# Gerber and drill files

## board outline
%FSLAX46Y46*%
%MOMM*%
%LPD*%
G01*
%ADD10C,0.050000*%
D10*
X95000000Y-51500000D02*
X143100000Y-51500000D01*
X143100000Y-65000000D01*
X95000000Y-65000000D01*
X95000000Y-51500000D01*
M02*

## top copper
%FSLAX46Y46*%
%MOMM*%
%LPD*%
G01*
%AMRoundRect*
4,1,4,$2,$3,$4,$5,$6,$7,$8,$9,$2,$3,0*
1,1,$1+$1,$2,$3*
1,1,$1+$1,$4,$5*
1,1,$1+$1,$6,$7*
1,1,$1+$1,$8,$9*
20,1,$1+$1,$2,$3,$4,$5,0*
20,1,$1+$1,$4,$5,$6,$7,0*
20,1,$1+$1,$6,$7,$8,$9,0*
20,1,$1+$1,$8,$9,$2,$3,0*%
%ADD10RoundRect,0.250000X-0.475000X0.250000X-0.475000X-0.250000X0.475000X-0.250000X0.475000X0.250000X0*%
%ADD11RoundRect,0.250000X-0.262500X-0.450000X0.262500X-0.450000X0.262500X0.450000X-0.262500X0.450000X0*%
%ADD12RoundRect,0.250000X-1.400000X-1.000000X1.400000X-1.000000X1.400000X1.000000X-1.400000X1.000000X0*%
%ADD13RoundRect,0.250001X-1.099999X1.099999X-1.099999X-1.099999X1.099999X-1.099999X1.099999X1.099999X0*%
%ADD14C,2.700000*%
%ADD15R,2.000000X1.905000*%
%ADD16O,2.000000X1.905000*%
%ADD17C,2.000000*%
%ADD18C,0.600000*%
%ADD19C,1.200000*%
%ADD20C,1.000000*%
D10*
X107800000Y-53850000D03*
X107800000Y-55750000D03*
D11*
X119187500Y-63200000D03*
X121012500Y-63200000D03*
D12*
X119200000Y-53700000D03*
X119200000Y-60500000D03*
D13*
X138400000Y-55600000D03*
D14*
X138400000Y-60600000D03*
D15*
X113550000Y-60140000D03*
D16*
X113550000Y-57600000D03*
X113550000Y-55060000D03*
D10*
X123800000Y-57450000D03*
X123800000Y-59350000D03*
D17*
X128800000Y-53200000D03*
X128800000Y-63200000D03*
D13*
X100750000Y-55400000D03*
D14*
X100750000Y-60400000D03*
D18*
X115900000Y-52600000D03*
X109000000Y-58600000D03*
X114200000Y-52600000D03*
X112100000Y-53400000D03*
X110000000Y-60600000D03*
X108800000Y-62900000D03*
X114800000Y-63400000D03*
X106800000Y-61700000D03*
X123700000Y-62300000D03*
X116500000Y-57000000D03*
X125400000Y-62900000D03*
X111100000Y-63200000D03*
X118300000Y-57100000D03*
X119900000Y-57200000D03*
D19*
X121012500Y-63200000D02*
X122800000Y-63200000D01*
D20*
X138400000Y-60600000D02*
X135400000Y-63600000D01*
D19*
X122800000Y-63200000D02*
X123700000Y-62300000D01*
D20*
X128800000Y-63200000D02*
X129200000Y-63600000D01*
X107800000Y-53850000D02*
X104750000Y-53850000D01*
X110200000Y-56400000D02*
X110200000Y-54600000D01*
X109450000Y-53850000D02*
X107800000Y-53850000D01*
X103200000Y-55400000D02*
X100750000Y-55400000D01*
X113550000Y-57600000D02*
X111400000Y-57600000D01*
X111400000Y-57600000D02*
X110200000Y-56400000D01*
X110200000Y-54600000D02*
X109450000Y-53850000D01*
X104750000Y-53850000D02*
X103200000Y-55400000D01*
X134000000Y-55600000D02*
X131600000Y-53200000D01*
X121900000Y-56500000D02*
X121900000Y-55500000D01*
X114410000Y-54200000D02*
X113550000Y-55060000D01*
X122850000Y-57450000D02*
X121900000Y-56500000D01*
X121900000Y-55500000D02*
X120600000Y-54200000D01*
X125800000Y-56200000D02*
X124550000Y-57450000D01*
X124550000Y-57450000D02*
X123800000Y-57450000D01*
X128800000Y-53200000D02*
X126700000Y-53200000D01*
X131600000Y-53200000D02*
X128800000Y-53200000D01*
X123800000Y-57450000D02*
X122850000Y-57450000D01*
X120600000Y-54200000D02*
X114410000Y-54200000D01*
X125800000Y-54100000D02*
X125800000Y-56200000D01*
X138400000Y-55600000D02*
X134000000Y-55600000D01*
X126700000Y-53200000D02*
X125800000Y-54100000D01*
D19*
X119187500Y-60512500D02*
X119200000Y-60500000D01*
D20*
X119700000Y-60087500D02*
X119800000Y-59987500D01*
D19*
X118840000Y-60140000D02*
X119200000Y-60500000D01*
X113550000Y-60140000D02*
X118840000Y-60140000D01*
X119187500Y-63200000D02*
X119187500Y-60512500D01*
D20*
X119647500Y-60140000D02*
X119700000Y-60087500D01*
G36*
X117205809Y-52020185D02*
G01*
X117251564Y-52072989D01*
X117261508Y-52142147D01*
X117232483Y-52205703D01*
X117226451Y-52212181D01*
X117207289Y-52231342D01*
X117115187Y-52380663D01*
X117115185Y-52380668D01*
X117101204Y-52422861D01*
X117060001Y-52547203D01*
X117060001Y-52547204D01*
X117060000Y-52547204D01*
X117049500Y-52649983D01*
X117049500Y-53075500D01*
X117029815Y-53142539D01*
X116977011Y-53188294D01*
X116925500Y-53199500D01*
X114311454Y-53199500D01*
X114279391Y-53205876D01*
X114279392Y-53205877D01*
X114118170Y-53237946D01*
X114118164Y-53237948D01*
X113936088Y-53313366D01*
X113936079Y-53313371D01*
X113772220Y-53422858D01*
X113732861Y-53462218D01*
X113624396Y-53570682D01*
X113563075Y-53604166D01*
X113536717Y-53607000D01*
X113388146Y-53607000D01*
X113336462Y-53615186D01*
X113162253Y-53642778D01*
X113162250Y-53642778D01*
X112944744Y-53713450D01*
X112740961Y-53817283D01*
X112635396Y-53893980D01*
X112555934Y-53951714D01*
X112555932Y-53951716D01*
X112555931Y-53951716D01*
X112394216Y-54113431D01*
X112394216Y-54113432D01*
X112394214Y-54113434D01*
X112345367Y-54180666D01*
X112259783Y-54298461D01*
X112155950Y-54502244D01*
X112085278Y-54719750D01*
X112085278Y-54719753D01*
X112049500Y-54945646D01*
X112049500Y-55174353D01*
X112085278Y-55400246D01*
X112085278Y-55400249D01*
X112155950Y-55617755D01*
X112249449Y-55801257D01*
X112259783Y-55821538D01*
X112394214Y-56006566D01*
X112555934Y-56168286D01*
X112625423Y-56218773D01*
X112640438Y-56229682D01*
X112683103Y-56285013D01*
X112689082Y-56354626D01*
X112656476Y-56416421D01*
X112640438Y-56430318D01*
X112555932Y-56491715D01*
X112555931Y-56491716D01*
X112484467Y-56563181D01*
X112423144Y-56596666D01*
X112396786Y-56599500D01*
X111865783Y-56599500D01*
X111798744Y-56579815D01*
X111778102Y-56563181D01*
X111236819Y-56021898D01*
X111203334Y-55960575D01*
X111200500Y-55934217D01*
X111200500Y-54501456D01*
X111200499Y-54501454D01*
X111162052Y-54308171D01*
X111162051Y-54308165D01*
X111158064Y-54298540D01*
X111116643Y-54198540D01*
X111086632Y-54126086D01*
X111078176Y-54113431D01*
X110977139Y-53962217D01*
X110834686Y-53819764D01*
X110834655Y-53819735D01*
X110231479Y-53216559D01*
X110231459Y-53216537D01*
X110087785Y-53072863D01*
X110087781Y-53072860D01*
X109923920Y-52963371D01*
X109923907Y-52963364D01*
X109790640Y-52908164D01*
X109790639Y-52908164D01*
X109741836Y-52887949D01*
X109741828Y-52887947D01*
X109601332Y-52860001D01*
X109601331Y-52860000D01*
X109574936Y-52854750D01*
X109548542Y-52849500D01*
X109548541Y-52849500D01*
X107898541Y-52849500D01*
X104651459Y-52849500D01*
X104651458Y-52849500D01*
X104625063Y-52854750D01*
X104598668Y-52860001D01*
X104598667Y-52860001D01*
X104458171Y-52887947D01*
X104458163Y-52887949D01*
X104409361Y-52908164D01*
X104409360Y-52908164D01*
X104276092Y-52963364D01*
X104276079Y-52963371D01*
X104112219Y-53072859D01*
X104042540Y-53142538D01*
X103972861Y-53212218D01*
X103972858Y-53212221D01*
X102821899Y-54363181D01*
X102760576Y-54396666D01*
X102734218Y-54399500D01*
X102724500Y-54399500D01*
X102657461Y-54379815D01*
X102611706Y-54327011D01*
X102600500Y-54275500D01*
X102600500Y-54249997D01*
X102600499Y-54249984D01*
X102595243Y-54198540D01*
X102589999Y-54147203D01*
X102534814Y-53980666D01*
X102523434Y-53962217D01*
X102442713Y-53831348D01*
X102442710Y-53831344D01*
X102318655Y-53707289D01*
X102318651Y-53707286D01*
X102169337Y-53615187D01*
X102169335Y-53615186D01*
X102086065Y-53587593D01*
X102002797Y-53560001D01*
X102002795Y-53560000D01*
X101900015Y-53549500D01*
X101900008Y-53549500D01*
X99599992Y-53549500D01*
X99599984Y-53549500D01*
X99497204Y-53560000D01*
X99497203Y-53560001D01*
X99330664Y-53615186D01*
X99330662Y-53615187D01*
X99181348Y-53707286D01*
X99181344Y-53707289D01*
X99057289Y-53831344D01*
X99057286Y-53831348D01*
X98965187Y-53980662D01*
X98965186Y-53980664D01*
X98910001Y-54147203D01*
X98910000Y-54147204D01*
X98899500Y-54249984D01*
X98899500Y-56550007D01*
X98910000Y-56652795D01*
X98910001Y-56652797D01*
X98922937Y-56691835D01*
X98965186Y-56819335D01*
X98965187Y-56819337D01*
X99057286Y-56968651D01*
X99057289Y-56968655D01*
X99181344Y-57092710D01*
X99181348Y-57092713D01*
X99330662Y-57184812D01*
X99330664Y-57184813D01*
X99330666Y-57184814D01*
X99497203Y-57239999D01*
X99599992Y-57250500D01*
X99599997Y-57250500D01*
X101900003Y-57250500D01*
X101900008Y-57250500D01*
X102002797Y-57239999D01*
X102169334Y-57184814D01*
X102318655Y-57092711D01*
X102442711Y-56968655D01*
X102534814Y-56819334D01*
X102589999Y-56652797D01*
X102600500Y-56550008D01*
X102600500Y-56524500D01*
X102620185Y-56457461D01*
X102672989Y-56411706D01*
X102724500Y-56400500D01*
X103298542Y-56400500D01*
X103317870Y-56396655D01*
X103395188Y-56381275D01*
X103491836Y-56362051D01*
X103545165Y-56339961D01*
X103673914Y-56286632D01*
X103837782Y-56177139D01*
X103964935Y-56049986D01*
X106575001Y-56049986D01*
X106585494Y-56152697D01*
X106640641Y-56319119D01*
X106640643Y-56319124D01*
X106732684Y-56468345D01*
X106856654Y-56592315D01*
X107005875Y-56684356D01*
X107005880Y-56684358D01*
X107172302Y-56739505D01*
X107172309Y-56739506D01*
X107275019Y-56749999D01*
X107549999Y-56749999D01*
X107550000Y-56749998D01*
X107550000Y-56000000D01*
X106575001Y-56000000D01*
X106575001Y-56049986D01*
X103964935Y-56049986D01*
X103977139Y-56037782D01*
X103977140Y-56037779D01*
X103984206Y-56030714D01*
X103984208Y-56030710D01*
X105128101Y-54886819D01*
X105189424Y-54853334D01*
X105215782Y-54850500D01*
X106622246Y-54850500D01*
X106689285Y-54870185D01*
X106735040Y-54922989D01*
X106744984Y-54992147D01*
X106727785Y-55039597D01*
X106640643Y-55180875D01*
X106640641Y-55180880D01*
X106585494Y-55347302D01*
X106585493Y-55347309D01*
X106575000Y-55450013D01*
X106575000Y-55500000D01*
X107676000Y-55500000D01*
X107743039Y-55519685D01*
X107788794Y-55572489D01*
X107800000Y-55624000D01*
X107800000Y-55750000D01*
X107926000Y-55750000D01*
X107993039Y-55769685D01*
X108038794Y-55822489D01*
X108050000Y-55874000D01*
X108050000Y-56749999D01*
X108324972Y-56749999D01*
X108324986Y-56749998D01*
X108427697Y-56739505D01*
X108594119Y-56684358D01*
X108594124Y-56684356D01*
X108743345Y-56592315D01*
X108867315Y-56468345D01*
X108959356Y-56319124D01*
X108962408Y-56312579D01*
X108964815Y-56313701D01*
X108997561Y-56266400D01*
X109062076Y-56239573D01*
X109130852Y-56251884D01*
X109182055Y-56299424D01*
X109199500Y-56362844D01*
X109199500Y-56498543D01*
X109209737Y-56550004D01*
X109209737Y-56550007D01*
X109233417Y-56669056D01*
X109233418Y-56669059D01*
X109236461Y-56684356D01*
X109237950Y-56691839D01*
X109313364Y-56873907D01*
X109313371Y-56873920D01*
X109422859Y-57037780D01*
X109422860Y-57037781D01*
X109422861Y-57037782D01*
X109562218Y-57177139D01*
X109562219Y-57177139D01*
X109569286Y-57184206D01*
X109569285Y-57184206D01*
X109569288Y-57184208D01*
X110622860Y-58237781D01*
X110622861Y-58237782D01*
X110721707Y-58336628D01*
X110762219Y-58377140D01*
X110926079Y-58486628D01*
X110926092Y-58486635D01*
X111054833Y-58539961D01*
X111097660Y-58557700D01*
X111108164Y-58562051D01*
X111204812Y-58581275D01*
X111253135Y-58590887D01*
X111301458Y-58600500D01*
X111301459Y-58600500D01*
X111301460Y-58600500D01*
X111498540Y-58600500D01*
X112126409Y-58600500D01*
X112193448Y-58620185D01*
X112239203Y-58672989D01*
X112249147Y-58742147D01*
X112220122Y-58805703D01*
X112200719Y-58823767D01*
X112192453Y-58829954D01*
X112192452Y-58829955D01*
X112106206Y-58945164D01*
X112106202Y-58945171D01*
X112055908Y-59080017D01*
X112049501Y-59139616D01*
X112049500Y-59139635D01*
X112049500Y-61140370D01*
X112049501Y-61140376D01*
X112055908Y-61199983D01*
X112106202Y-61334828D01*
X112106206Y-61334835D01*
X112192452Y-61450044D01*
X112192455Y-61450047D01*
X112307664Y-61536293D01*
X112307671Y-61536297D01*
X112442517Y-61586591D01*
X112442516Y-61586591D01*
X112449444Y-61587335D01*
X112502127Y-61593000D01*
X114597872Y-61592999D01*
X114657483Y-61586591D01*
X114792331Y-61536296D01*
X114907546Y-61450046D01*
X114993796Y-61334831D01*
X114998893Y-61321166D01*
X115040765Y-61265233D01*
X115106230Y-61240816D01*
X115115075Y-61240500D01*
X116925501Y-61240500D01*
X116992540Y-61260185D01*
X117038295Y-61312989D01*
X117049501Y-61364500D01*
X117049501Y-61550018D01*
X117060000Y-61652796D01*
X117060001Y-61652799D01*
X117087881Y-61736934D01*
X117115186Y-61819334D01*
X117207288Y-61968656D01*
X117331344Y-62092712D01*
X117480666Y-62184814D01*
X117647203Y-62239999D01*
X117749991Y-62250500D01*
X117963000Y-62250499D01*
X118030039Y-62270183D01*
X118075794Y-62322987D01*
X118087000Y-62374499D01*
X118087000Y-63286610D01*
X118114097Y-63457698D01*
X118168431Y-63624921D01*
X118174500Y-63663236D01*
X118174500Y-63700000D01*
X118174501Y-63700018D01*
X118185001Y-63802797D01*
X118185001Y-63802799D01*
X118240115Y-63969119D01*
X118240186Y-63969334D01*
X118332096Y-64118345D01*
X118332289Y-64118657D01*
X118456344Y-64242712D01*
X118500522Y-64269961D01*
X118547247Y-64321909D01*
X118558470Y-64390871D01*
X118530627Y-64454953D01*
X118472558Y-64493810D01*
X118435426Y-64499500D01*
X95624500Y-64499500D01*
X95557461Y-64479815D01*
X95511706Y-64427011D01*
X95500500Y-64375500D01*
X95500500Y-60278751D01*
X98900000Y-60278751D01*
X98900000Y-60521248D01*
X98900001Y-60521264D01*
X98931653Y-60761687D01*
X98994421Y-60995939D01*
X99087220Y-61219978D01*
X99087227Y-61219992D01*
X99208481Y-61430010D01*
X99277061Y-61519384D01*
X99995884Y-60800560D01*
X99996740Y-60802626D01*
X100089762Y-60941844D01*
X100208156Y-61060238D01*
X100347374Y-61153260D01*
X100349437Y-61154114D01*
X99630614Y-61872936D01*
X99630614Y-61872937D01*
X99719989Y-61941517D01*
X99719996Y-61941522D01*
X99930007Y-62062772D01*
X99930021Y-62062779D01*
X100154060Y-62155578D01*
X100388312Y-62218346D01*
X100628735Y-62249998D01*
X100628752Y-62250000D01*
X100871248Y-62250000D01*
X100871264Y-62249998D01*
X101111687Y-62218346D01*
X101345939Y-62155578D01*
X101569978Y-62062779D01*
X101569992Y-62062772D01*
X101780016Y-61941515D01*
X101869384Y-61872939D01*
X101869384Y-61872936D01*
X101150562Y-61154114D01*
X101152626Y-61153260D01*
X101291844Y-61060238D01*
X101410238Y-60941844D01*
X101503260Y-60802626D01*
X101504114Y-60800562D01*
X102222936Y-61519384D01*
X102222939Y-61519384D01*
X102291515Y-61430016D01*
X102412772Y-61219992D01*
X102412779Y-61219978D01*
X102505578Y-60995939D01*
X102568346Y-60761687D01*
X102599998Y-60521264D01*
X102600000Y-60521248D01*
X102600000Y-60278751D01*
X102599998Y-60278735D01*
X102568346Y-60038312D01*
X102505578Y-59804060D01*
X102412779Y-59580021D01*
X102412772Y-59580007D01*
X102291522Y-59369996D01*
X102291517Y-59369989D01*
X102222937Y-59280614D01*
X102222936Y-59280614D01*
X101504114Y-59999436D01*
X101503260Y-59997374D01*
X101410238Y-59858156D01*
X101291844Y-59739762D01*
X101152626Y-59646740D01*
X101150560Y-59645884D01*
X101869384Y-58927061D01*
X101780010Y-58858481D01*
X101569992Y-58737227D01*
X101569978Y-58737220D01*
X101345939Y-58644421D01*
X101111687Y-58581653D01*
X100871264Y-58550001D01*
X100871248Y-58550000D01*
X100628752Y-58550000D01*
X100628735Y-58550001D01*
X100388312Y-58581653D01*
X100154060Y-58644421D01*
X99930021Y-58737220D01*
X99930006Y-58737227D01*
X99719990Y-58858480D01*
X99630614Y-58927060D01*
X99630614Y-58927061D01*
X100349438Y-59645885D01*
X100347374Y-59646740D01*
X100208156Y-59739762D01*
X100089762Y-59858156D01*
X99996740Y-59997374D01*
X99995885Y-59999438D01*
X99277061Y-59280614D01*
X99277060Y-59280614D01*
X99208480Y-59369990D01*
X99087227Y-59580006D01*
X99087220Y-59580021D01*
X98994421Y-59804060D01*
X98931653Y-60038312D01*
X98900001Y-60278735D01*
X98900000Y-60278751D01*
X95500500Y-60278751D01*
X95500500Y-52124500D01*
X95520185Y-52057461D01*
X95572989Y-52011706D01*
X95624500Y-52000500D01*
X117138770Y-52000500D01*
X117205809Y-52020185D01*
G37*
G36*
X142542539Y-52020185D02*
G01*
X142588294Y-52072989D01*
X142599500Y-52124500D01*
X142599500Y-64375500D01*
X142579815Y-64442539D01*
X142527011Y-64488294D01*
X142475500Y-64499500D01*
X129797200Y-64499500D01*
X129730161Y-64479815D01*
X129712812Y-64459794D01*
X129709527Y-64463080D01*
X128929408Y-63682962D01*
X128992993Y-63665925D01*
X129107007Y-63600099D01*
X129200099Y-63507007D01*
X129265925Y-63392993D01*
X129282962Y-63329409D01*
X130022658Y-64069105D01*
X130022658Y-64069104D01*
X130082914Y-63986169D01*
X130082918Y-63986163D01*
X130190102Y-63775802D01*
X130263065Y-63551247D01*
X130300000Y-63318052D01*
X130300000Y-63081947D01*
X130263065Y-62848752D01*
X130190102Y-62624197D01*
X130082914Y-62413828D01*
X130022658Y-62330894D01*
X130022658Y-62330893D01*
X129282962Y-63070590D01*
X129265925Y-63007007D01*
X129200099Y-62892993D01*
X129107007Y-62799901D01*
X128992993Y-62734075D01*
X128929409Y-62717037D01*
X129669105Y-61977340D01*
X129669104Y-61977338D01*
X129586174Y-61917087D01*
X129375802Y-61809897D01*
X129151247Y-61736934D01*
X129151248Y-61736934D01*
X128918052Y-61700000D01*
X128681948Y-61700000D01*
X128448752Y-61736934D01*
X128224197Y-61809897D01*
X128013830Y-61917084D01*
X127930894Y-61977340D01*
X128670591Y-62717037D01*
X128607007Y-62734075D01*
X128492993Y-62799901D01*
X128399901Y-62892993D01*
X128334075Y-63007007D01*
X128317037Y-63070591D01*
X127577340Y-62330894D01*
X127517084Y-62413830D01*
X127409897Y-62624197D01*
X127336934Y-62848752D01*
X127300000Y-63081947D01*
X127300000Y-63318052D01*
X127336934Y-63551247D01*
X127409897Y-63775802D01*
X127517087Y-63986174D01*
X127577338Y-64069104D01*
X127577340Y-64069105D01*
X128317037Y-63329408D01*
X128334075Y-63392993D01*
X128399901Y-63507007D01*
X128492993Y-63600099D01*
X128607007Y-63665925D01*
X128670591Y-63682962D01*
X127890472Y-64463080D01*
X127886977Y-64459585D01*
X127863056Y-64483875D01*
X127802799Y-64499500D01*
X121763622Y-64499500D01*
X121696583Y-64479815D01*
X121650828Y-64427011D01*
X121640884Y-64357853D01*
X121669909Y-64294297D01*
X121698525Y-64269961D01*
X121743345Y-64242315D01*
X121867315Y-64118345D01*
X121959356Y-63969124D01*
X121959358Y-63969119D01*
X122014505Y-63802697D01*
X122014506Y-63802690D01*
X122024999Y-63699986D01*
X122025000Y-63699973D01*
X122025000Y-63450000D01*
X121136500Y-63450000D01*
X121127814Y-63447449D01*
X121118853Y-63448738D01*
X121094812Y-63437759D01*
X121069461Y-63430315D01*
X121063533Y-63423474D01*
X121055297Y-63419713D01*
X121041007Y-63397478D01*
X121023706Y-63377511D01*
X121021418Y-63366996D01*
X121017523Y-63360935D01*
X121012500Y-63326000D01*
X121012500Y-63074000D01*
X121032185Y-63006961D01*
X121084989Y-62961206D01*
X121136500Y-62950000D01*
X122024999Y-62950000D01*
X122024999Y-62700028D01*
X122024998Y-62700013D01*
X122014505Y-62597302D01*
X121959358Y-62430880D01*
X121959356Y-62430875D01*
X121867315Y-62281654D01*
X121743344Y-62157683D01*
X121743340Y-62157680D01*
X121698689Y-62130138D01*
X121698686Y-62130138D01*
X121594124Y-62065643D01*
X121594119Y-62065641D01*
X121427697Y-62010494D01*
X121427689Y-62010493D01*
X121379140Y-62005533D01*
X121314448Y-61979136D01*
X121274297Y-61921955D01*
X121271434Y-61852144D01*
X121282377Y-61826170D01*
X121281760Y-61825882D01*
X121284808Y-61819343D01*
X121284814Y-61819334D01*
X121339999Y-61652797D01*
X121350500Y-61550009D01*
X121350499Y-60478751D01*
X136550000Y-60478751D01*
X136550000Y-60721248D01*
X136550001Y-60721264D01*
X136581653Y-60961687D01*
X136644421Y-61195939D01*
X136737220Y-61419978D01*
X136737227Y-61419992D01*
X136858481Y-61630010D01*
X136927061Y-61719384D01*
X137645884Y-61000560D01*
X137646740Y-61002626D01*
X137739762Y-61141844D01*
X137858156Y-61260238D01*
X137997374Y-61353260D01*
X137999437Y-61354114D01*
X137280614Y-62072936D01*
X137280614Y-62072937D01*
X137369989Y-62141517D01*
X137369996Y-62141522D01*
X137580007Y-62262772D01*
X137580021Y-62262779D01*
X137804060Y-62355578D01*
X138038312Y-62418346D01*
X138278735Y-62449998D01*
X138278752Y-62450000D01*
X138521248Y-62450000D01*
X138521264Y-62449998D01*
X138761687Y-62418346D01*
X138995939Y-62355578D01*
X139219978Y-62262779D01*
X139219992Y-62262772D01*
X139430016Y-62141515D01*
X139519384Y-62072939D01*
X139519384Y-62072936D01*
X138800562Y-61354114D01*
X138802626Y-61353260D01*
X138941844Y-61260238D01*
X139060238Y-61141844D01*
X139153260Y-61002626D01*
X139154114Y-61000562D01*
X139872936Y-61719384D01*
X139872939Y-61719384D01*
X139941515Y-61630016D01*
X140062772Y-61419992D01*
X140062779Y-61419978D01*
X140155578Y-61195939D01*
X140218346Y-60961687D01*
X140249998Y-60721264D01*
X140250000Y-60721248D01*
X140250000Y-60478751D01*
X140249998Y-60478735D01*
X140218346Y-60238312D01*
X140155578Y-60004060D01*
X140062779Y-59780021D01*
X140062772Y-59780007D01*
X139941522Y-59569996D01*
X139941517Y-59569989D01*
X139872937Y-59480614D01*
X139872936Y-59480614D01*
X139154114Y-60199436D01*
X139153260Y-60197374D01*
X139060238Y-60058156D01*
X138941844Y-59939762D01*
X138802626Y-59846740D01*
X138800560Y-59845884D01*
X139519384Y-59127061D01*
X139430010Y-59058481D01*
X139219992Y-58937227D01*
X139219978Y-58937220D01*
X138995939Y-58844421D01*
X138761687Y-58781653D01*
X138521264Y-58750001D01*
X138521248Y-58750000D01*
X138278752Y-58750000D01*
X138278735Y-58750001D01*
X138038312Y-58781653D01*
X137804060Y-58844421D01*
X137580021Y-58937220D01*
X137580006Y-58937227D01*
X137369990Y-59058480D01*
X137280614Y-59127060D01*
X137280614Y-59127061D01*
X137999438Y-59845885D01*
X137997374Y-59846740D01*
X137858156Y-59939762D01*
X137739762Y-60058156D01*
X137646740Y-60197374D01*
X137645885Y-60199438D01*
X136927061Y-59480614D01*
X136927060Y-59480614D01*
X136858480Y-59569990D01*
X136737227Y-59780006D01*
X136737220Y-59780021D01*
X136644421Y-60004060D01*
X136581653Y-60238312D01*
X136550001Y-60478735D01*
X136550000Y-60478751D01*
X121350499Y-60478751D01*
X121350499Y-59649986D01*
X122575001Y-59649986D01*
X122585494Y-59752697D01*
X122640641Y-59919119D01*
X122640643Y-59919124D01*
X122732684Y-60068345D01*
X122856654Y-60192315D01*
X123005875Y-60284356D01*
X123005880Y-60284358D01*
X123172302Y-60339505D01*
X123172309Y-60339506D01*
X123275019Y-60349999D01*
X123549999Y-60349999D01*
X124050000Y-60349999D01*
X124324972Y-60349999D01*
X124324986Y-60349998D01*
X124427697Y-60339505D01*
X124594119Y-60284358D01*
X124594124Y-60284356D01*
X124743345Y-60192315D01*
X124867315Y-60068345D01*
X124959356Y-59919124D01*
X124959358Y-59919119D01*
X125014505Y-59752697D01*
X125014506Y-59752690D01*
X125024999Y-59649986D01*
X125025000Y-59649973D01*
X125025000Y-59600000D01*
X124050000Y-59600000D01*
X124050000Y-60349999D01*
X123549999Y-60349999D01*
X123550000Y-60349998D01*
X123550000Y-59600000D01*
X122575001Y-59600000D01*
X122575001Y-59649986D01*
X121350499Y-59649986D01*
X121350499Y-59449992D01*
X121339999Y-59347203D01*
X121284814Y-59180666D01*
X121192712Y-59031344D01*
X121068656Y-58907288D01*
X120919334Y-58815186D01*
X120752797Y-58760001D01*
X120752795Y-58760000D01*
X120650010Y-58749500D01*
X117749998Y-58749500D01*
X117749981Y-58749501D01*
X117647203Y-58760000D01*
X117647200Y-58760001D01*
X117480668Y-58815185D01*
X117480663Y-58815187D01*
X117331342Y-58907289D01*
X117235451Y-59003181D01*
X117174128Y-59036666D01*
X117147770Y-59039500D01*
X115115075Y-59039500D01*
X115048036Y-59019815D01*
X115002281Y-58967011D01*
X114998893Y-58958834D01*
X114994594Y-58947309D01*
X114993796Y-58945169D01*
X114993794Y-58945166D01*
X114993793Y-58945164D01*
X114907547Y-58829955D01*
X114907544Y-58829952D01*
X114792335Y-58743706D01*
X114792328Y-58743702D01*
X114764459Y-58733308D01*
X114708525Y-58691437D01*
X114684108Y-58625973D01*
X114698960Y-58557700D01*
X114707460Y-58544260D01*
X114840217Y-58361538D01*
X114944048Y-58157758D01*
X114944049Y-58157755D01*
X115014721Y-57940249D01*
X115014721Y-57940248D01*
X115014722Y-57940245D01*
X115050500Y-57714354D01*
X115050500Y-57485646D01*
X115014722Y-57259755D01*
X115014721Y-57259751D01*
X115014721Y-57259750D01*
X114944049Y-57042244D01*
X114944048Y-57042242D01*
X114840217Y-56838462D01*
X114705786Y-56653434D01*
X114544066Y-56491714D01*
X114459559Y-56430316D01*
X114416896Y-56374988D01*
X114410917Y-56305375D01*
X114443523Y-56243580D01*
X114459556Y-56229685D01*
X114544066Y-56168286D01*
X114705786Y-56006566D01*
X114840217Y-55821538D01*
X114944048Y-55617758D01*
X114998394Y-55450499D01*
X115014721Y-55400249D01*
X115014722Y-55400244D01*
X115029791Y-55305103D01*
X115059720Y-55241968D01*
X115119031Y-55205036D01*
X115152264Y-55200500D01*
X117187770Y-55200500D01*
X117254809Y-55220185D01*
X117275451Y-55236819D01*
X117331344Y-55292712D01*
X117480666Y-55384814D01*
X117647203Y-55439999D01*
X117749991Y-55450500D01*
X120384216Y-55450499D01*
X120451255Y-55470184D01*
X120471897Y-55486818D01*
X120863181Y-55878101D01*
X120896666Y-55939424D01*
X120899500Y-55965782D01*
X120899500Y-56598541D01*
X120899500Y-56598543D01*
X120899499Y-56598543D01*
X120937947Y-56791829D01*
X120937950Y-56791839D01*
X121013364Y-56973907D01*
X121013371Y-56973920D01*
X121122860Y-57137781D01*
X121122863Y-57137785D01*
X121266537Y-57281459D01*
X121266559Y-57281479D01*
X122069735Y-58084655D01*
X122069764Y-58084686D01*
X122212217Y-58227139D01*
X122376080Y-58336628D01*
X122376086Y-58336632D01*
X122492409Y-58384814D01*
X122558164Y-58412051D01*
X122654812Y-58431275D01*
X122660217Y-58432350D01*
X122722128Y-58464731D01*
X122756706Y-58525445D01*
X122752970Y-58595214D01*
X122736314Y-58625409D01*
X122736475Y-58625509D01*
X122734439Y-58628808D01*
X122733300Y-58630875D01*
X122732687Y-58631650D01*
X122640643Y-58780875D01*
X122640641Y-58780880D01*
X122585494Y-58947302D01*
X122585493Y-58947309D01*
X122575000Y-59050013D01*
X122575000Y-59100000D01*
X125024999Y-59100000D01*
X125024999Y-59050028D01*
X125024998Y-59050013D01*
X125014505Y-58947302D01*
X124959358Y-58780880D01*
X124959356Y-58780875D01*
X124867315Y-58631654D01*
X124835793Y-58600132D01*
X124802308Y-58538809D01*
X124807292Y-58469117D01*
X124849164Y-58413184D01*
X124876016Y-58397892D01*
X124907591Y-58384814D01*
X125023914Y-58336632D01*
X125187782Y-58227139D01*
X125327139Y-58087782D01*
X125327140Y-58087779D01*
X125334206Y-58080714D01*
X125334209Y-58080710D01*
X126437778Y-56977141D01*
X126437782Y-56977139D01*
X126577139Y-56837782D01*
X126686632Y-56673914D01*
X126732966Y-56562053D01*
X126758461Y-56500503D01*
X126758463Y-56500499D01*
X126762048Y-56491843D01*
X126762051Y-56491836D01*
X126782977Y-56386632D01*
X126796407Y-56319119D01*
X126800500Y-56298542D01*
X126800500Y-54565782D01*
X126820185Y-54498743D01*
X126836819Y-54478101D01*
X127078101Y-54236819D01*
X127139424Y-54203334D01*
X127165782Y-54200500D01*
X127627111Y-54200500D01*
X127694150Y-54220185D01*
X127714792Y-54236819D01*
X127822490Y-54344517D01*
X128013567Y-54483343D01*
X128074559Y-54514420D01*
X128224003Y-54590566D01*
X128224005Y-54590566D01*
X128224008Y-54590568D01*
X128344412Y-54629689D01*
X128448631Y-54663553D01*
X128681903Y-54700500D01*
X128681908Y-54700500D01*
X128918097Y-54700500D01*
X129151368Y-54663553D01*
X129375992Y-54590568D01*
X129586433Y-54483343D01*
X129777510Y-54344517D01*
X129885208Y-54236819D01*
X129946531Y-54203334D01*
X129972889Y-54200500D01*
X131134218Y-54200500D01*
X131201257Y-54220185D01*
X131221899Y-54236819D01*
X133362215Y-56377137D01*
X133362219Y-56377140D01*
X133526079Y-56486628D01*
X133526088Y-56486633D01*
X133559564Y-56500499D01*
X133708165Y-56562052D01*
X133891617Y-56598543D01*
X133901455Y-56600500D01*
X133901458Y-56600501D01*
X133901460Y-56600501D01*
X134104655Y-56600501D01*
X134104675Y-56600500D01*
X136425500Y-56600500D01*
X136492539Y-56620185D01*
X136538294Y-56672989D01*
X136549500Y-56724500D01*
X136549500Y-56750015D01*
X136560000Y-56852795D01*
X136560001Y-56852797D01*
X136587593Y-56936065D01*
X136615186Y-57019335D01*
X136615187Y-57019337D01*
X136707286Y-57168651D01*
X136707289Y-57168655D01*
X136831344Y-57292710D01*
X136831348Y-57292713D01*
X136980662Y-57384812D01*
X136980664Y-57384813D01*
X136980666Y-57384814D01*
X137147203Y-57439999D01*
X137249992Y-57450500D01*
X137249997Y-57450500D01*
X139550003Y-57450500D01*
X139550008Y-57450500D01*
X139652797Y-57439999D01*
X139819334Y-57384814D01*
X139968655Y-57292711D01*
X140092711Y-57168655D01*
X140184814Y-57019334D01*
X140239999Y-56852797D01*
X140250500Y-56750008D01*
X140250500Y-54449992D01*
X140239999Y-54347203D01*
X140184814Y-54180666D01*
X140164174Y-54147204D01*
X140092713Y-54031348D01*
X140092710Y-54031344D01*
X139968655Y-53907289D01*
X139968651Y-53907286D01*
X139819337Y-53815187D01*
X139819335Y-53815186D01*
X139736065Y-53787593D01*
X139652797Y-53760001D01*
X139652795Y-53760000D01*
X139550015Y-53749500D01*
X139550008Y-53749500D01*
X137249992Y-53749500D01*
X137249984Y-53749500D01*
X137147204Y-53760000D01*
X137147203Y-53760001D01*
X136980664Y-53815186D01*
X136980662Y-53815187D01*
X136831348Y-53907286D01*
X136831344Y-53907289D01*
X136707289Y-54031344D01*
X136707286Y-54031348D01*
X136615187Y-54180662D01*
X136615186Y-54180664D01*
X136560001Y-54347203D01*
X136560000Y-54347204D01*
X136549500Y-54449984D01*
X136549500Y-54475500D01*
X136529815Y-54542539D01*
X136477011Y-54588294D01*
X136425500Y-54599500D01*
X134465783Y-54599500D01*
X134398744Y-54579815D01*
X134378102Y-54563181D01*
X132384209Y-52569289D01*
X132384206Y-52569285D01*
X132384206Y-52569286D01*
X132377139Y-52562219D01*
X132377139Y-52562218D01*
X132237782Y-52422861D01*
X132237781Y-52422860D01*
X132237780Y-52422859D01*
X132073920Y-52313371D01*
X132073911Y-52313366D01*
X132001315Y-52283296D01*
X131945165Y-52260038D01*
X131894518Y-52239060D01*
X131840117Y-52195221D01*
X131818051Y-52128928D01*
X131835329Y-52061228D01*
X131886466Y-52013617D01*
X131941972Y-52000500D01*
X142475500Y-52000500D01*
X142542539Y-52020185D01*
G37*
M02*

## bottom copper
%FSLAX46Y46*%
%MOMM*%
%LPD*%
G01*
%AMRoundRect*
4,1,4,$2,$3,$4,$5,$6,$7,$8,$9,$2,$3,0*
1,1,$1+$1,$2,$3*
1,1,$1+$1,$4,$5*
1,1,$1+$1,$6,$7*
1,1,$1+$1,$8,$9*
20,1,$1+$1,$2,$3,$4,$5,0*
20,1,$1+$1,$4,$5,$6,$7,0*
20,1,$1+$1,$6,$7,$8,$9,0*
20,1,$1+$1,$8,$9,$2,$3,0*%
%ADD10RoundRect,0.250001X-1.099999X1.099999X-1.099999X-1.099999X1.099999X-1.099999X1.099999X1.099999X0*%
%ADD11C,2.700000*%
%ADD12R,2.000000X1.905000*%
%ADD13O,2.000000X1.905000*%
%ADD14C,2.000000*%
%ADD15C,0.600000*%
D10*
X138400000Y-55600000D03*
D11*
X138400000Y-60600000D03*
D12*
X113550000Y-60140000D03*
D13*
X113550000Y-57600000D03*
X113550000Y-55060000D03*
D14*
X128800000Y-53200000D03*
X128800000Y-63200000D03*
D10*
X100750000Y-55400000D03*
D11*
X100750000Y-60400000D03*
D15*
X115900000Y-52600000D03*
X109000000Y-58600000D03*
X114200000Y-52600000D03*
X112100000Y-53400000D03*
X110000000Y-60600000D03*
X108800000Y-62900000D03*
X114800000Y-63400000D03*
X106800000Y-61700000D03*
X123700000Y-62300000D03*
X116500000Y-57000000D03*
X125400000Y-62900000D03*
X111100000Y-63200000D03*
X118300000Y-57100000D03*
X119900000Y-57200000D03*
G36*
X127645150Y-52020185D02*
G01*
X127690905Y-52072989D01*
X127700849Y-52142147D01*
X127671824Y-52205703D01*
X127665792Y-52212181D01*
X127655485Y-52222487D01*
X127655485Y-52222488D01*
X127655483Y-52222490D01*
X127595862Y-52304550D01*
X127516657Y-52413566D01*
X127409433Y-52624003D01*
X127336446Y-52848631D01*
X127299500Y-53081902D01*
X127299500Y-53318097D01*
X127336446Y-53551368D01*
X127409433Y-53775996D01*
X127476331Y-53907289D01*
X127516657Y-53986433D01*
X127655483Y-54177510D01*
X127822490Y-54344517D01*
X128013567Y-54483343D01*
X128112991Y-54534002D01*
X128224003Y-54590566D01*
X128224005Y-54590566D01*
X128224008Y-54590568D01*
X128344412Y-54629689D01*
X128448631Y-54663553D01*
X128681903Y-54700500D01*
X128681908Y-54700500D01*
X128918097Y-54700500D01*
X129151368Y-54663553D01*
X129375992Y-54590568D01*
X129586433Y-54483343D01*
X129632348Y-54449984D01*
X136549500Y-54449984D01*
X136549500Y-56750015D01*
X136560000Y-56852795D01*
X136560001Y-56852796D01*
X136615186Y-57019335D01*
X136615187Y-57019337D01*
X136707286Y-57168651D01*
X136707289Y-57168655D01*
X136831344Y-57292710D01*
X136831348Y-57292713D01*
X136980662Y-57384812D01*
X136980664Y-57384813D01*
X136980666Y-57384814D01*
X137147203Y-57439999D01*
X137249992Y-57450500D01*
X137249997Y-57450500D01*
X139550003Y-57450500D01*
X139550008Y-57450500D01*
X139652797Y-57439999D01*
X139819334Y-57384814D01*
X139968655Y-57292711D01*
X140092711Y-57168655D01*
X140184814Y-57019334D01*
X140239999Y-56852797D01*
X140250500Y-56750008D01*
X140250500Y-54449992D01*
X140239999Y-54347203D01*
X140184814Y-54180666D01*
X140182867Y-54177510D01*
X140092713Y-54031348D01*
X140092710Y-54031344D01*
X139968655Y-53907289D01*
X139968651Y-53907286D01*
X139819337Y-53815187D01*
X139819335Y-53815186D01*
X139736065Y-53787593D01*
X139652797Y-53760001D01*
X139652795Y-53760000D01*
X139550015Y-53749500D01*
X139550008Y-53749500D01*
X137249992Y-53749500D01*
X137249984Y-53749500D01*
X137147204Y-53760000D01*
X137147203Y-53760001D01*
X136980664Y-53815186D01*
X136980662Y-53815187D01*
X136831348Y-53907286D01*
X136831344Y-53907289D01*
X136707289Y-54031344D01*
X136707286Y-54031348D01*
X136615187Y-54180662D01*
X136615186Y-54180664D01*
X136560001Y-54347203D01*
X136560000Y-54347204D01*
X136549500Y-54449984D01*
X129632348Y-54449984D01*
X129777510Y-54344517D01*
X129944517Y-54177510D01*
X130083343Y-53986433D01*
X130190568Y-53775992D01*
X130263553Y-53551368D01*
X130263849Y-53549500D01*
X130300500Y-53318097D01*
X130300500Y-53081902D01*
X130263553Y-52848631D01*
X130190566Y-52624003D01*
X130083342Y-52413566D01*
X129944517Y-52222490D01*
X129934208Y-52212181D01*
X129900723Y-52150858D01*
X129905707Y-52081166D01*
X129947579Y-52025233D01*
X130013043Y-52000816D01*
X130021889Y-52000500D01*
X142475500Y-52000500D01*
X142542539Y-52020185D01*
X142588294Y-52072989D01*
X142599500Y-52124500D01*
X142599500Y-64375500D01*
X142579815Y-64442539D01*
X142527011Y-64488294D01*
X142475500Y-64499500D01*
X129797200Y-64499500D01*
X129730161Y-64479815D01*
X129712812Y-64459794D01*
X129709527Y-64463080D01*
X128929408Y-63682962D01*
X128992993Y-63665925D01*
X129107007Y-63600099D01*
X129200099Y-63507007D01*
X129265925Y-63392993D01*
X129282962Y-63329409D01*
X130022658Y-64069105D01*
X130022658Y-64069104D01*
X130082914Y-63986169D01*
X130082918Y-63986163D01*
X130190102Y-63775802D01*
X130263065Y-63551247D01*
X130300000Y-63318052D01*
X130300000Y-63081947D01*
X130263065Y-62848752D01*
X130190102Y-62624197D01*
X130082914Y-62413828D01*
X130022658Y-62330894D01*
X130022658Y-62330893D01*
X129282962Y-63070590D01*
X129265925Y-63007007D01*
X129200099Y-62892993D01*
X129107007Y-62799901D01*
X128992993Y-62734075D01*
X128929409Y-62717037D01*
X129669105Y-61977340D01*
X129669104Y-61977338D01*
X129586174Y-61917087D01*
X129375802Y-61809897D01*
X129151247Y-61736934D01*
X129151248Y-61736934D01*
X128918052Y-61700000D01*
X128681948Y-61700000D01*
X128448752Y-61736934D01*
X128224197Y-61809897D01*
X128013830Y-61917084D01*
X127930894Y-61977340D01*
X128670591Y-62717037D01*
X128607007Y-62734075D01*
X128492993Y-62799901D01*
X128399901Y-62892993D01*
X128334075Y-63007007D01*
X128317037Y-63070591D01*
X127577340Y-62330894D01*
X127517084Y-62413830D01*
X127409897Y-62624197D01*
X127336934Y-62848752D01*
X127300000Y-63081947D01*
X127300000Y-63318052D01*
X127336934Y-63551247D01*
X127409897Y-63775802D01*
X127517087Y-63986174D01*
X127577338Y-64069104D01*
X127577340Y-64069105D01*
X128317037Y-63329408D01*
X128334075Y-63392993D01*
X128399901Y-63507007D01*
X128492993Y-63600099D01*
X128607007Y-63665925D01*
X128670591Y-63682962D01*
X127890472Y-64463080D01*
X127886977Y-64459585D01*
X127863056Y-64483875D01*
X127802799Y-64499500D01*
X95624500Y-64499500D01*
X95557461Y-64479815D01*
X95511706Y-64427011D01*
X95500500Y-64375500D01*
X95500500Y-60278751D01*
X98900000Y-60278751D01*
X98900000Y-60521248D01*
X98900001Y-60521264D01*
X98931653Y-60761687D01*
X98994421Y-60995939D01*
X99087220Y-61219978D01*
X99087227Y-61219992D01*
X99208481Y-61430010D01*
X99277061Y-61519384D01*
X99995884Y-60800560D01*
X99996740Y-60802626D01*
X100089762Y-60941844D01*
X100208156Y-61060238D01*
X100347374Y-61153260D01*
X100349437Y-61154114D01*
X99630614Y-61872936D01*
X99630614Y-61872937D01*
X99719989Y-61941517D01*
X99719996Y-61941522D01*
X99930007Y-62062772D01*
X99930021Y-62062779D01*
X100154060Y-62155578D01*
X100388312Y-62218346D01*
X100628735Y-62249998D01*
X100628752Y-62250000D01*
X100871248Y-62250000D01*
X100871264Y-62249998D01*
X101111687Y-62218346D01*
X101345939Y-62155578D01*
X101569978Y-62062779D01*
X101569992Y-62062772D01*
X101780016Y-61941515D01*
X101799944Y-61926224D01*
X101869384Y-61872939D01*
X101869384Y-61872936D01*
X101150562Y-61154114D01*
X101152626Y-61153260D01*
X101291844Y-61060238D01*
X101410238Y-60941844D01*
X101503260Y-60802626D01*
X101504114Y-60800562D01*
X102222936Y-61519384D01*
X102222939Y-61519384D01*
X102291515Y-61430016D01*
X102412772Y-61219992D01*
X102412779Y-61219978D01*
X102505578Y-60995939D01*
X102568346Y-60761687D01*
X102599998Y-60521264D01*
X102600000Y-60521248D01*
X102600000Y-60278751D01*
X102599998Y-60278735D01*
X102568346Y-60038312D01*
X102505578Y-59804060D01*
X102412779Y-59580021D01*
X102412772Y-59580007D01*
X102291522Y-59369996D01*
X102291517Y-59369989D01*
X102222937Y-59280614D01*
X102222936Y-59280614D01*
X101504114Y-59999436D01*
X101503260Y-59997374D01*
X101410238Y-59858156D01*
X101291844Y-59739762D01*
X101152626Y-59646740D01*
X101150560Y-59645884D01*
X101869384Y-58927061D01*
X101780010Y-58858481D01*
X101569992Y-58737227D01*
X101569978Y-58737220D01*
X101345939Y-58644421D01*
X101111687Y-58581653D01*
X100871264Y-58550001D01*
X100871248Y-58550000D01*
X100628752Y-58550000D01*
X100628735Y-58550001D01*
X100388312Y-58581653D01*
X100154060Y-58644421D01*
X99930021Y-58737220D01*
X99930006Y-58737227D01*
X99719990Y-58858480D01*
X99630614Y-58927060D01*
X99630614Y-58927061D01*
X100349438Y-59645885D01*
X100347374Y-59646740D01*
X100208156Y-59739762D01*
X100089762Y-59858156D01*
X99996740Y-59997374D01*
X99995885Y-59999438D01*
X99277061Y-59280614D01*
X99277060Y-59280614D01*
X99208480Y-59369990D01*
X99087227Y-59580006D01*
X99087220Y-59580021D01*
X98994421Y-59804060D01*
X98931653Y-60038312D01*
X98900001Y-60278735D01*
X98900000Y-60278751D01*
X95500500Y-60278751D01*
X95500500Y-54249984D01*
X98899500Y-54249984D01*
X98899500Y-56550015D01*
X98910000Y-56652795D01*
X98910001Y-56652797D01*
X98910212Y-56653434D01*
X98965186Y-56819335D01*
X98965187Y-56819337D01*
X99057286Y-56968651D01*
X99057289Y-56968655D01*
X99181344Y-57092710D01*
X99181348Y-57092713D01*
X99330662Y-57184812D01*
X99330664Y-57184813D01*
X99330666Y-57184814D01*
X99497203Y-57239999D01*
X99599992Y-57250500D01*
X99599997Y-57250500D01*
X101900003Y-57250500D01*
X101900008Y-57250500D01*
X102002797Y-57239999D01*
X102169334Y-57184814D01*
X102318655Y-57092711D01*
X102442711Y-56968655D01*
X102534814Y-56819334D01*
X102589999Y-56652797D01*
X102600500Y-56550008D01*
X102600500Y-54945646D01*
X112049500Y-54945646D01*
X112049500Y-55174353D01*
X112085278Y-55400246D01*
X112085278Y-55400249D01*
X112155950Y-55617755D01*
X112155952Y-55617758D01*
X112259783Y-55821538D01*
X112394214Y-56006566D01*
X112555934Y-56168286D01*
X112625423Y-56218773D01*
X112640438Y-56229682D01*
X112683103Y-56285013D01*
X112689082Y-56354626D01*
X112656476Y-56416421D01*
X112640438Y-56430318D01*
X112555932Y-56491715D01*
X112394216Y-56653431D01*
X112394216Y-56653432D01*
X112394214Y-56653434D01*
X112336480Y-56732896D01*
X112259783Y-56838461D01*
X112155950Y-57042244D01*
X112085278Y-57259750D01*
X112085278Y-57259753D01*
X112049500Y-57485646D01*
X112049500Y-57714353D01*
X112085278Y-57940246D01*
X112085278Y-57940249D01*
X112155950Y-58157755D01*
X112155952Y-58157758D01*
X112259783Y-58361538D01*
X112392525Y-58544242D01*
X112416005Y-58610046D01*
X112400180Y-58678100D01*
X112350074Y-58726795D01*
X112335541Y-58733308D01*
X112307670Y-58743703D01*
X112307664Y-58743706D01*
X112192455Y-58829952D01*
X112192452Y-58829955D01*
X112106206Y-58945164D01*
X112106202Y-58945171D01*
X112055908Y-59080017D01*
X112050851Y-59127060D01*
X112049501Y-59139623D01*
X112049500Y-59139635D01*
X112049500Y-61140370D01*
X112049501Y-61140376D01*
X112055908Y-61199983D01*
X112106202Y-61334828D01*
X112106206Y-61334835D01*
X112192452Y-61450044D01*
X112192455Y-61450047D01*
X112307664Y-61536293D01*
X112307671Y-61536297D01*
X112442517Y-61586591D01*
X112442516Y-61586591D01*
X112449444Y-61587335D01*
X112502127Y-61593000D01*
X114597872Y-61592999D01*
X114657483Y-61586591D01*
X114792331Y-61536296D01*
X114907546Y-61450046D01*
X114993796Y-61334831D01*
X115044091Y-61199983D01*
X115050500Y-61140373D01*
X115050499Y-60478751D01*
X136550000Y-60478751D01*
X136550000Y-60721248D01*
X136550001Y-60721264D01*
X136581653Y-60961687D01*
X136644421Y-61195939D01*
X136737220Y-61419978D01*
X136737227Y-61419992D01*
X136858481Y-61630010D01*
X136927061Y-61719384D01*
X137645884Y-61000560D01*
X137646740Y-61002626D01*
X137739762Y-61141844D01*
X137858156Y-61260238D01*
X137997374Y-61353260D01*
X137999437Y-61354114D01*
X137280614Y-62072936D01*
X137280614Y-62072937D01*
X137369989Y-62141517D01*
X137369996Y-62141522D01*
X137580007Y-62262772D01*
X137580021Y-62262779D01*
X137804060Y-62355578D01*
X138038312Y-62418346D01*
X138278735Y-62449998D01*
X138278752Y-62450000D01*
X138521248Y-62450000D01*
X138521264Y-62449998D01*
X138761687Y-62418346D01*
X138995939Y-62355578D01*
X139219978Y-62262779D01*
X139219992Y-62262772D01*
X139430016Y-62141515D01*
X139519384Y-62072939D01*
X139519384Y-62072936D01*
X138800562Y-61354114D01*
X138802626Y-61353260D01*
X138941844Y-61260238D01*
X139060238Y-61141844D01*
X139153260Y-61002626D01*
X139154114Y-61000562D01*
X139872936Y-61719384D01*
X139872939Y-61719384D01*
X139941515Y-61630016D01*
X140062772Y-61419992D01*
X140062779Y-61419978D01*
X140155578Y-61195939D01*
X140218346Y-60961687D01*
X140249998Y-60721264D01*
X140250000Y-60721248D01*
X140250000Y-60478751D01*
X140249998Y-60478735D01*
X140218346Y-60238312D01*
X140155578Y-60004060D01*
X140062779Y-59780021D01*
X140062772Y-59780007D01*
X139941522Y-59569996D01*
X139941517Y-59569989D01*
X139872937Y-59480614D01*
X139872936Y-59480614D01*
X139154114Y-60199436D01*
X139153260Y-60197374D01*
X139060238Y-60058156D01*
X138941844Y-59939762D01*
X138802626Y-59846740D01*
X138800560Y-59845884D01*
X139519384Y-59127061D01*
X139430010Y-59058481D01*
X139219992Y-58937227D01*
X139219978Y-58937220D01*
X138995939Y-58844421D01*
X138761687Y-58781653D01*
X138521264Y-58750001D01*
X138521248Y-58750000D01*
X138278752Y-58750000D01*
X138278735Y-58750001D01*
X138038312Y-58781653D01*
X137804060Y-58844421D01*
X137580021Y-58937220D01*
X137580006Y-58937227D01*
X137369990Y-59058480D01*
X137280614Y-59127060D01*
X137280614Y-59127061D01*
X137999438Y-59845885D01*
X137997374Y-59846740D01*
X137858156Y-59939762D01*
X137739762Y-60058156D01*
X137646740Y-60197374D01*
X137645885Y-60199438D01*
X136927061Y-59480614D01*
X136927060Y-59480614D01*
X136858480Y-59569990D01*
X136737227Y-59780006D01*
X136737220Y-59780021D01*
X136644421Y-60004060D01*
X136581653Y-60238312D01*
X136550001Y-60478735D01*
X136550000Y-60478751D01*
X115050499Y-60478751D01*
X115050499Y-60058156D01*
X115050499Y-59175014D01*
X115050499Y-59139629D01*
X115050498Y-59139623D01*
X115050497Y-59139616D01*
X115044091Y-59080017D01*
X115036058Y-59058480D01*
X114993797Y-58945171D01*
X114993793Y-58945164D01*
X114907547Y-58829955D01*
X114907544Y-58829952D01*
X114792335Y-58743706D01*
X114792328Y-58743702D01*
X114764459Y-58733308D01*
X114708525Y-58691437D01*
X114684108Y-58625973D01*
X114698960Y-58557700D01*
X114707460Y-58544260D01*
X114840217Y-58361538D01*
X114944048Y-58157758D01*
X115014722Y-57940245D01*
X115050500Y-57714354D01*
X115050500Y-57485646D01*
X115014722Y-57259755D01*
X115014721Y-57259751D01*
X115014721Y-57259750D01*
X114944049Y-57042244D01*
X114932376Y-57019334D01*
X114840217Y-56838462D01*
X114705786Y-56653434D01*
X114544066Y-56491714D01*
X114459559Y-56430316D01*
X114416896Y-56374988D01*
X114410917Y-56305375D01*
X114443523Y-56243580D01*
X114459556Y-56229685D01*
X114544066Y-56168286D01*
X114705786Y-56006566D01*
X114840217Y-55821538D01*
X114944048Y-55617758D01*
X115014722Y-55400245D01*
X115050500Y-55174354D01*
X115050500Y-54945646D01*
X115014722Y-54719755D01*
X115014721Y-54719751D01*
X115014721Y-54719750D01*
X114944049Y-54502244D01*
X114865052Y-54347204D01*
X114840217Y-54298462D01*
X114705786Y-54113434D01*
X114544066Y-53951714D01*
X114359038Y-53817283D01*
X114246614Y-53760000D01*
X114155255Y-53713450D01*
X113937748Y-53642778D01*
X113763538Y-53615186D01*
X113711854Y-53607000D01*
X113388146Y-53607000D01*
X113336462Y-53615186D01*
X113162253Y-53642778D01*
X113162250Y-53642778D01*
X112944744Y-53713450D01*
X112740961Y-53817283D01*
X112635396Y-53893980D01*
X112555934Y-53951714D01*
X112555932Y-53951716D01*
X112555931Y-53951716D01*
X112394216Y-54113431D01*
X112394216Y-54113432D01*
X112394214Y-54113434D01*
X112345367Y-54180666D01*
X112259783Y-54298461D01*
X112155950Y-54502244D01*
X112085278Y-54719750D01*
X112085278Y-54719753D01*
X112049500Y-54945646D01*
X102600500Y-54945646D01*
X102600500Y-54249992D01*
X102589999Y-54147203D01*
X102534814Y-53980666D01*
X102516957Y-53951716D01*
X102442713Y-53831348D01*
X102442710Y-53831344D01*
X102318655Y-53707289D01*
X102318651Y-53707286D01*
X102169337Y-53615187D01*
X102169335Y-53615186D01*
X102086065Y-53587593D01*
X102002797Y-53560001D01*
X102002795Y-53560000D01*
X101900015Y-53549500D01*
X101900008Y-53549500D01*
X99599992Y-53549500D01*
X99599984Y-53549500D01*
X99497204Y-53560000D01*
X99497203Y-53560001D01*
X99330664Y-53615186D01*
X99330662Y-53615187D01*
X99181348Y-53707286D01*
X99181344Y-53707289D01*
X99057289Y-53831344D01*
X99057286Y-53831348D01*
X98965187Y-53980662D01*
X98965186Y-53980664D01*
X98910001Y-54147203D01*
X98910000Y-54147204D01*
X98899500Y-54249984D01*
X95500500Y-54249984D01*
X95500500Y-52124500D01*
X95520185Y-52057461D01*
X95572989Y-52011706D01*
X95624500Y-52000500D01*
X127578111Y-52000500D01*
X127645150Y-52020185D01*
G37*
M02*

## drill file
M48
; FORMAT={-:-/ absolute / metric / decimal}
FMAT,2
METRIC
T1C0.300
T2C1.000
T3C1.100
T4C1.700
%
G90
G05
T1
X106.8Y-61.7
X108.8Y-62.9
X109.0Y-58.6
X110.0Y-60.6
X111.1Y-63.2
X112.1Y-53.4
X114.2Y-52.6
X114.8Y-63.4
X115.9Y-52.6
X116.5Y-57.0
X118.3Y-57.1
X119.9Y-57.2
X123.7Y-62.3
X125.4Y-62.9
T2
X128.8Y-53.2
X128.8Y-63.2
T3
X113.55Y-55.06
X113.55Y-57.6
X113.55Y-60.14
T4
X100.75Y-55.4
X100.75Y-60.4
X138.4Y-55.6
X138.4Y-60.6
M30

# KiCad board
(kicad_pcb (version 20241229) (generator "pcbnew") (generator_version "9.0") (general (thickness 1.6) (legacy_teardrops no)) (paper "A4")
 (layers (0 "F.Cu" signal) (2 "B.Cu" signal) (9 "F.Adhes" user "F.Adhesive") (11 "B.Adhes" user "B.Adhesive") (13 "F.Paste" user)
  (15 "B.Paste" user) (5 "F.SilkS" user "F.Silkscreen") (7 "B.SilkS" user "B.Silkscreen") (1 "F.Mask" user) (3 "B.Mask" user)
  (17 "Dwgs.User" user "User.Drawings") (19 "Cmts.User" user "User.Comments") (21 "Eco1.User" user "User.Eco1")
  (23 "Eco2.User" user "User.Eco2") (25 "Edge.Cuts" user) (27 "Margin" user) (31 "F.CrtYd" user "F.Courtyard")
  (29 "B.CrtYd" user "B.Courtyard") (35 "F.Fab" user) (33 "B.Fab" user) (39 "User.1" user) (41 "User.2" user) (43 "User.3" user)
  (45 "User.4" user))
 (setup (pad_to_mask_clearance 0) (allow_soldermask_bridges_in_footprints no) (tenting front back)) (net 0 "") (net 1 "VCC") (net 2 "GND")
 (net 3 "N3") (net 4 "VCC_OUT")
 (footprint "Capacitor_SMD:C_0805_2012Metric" (layer "F.Cu") (at 107.8 54.8 -90)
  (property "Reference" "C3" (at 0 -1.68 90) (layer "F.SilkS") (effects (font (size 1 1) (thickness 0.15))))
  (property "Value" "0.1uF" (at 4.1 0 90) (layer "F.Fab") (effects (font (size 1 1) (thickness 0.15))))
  (pad "1" smd roundrect (at -0.95 0 270) (size 1 1.45) (layers "F.Cu" "F.Mask" "F.Paste") (roundrect_rratio 0.25) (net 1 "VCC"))
  (pad "2" smd roundrect (at 0.95 0 270) (size 1 1.45) (layers "F.Cu" "F.Mask" "F.Paste") (roundrect_rratio 0.25) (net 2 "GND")))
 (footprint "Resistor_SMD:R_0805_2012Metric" (layer "F.Cu") (at 120.1 63.2)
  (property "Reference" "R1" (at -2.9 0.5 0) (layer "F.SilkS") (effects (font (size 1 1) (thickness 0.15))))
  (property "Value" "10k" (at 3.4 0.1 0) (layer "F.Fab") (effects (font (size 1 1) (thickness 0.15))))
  (pad "1" smd roundrect (at -0.9125 0) (size 1.025 1.4) (layers "F.Cu" "F.Mask" "F.Paste") (roundrect_rratio 0.243902) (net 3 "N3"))
  (pad "2" smd roundrect (at 0.9125 0) (size 1.025 1.4) (layers "F.Cu" "F.Mask" "F.Paste") (roundrect_rratio 0.243902) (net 2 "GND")))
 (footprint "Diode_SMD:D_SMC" (layer "F.Cu") (at 119.2 57.1 -90)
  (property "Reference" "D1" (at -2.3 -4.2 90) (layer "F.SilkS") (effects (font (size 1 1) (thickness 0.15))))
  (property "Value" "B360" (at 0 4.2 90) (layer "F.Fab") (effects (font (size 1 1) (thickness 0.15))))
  (pad "1" smd roundrect (at -3.4 0) (size 3.3 2.5) (layers "F.Cu" "F.Mask" "F.Paste") (roundrect_rratio 0.1) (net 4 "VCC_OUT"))
  (pad "2" smd roundrect (at 3.4 0) (size 3.3 2.5) (layers "F.Cu" "F.Mask" "F.Paste") (roundrect_rratio 0.1) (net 3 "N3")))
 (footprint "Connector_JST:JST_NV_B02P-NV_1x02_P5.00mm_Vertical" (layer "F.Cu") (at 138.4 55.6 -90)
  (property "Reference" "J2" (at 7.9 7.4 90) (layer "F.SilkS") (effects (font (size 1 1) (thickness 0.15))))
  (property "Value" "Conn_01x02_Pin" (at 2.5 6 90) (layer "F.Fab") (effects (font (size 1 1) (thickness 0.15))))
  (pad "1" thru_hole roundrect (at 0 0 270) (size 2.7 2.7) (drill 1.7) (layers "*.Cu" "*.Mask") (remove_unused_layers no)
   (roundrect_rratio 0.092593) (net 4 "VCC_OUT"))
  (pad "2" thru_hole circle (at 5 0 270) (size 2.7 2.7) (drill 1.7) (layers "*.Cu" "*.Mask") (remove_unused_layers no) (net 2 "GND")))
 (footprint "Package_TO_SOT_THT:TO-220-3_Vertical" (layer "F.Cu") (at 113.55 60.14 90)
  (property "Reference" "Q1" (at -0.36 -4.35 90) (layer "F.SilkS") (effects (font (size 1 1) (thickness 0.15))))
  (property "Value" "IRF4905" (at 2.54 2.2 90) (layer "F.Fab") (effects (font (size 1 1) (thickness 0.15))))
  (pad "1" thru_hole rect (at 0 0 90) (size 1.905 2) (drill 1.1) (layers "*.Cu" "*.Mask") (remove_unused_layers no) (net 3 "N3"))
  (pad "2" thru_hole oval (at 2.54 0 90) (size 1.905 2) (drill 1.1) (layers "*.Cu" "*.Mask") (remove_unused_layers no) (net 1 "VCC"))
  (pad "3" thru_hole oval (at 5.08 0 90) (size 1.905 2) (drill 1.1) (layers "*.Cu" "*.Mask") (remove_unused_layers no) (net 4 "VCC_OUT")))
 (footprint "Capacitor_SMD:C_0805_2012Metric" (layer "F.Cu") (at 123.8 58.4 -90)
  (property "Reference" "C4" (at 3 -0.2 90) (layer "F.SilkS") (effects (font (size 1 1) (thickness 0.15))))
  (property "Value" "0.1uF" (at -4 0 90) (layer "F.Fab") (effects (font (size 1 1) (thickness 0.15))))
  (pad "1" smd roundrect (at -0.95 0 270) (size 1 1.45) (layers "F.Cu" "F.Mask" "F.Paste") (roundrect_rratio 0.25) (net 4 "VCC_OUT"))
  (pad "2" smd roundrect (at 0.95 0 270) (size 1 1.45) (layers "F.Cu" "F.Mask" "F.Paste") (roundrect_rratio 0.25) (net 2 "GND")))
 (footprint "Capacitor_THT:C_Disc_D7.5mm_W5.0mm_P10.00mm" (layer "F.Cu") (at 128.8 53.2 -90)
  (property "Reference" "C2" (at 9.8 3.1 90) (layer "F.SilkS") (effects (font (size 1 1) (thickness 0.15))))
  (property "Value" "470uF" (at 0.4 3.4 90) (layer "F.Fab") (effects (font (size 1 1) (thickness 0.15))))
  (pad "1" thru_hole circle (at 0 0 270) (size 2 2) (drill 1) (layers "*.Cu" "*.Mask") (remove_unused_layers no) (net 4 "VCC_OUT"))
  (pad "2" thru_hole circle (at 10 0 270) (size 2 2) (drill 1) (layers "*.Cu" "*.Mask") (remove_unused_layers no) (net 2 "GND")))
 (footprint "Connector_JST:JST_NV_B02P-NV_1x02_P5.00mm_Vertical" (layer "F.Cu") (at 100.75 55.4 -90)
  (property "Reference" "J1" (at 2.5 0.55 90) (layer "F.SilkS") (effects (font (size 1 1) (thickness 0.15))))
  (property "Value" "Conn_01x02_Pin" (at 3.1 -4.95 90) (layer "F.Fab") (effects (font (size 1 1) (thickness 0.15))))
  (pad "1" thru_hole roundrect (at 0 0 270) (size 2.7 2.7) (drill 1.7) (layers "*.Cu" "*.Mask") (remove_unused_layers no)
   (roundrect_rratio 0.092593) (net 1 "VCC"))
  (pad "2" thru_hole circle (at 5 0 270) (size 2.7 2.7) (drill 1.7) (layers "*.Cu" "*.Mask") (remove_unused_layers no) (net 2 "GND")))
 (gr_rect (start 95 51.5) (end 143.1 65) (stroke (width 0.05) (type default)) (fill no) (layer "Edge.Cuts"))
 (segment (start 121.0125 63.2) (end 122.8 63.2) (width 1.2) (layer "F.Cu") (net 2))
 (segment (start 138.4 60.6) (end 135.4 63.6) (width 1) (layer "F.Cu") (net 2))
 (segment (start 122.8 63.2) (end 123.7 62.3) (width 1.2) (layer "F.Cu") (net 2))
 (segment (start 128.8 63.2) (end 129.2 63.6) (width 1) (layer "F.Cu") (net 2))
 (via (at 115.9 52.6) (size 0.6) (drill 0.3) (layers "F.Cu" "B.Cu") (free yes) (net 2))
 (via (at 109 58.6) (size 0.6) (drill 0.3) (layers "F.Cu" "B.Cu") (free yes) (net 2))
 (via (at 114.2 52.6) (size 0.6) (drill 0.3) (layers "F.Cu" "B.Cu") (free yes) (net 2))
 (via (at 112.1 53.4) (size 0.6) (drill 0.3) (layers "F.Cu" "B.Cu") (free yes) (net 2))
 (via (at 110 60.6) (size 0.6) (drill 0.3) (layers "F.Cu" "B.Cu") (free yes) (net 2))
 (via (at 108.8 62.9) (size 0.6) (drill 0.3) (layers "F.Cu" "B.Cu") (free yes) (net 2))
 (via (at 114.8 63.4) (size 0.6) (drill 0.3) (layers "F.Cu" "B.Cu") (free yes) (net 2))
 (via (at 106.8 61.7) (size 0.6) (drill 0.3) (layers "F.Cu" "B.Cu") (free yes) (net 2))
 (via (at 123.7 62.3) (size 0.6) (drill 0.3) (layers "F.Cu" "B.Cu") (free yes) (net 2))
 (via (at 116.5 57) (size 0.6) (drill 0.3) (layers "F.Cu" "B.Cu") (free yes) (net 2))
 (via (at 125.4 62.9) (size 0.6) (drill 0.3) (layers "F.Cu" "B.Cu") (free yes) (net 2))
 (via (at 111.1 63.2) (size 0.6) (drill 0.3) (layers "F.Cu" "B.Cu") (free yes) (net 2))
 (via (at 118.3 57.1) (size 0.6) (drill 0.3) (layers "F.Cu" "B.Cu") (free yes) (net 2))
 (via (at 119.9 57.2) (size 0.6) (drill 0.3) (layers "F.Cu" "B.Cu") (free yes) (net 2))
 (segment (start 107.8 53.85) (end 104.75 53.85) (width 1) (layer "F.Cu") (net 1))
 (segment (start 110.2 56.4) (end 110.2 54.6) (width 1) (layer "F.Cu") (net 1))
 (segment (start 109.45 53.85) (end 107.8 53.85) (width 1) (layer "F.Cu") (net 1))
 (segment (start 103.2 55.4) (end 100.75 55.4) (width 1) (layer "F.Cu") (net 1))
 (segment (start 113.55 57.6) (end 111.4 57.6) (width 1) (layer "F.Cu") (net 1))
 (segment (start 111.4 57.6) (end 110.2 56.4) (width 1) (layer "F.Cu") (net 1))
 (segment (start 110.2 54.6) (end 109.45 53.85) (width 1) (layer "F.Cu") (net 1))
 (segment (start 104.75 53.85) (end 103.2 55.4) (width 1) (layer "F.Cu") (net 1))
 (segment (start 134 55.6) (end 131.6 53.2) (width 1) (layer "F.Cu") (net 4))
 (segment (start 121.9 56.5) (end 121.9 55.5) (width 1) (layer "F.Cu") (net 4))
 (segment (start 114.41 54.2) (end 113.55 55.06) (width 1) (layer "F.Cu") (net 4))
 (segment (start 122.85 57.45) (end 121.9 56.5) (width 1) (layer "F.Cu") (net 4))
 (segment (start 121.9 55.5) (end 120.6 54.2) (width 1) (layer "F.Cu") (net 4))
 (segment (start 125.8 56.2) (end 124.55 57.45) (width 1) (layer "F.Cu") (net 4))
 (segment (start 124.55 57.45) (end 123.8 57.45) (width 1) (layer "F.Cu") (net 4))
 (segment (start 128.8 53.2) (end 126.7 53.2) (width 1) (layer "F.Cu") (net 4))
 (segment (start 131.6 53.2) (end 128.8 53.2) (width 1) (layer "F.Cu") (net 4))
 (segment (start 123.8 57.45) (end 122.85 57.45) (width 1) (layer "F.Cu") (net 4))
 (segment (start 120.6 54.2) (end 114.41 54.2) (width 1) (layer "F.Cu") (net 4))
 (segment (start 125.8 54.1) (end 125.8 56.2) (width 1) (layer "F.Cu") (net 4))
 (segment (start 138.4 55.6) (end 134 55.6) (width 1) (layer "F.Cu") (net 4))
 (segment (start 126.7 53.2) (end 125.8 54.1) (width 1) (layer "F.Cu") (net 4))
 (segment (start 119.1875 60.5125) (end 119.2 60.5) (width 1.2) (layer "F.Cu") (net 3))
 (segment (start 119.7 60.0875) (end 119.8 59.9875) (width 1) (layer "F.Cu") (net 3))
 (segment (start 118.84 60.14) (end 119.2 60.5) (width 1.2) (layer "F.Cu") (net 3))
 (segment (start 113.55 60.14) (end 118.84 60.14) (width 1.2) (layer "F.Cu") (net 3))
 (segment (start 119.1875 63.2) (end 119.1875 60.5125) (width 1.2) (layer "F.Cu") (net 3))
 (segment (start 119.6475 60.14) (end 119.7 60.0875) (width 1) (layer "F.Cu") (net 3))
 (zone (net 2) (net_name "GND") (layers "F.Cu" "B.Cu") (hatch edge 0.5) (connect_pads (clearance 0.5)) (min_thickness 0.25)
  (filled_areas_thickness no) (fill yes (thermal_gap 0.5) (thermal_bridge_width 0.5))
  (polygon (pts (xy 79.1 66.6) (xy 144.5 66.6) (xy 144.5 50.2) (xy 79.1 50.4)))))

